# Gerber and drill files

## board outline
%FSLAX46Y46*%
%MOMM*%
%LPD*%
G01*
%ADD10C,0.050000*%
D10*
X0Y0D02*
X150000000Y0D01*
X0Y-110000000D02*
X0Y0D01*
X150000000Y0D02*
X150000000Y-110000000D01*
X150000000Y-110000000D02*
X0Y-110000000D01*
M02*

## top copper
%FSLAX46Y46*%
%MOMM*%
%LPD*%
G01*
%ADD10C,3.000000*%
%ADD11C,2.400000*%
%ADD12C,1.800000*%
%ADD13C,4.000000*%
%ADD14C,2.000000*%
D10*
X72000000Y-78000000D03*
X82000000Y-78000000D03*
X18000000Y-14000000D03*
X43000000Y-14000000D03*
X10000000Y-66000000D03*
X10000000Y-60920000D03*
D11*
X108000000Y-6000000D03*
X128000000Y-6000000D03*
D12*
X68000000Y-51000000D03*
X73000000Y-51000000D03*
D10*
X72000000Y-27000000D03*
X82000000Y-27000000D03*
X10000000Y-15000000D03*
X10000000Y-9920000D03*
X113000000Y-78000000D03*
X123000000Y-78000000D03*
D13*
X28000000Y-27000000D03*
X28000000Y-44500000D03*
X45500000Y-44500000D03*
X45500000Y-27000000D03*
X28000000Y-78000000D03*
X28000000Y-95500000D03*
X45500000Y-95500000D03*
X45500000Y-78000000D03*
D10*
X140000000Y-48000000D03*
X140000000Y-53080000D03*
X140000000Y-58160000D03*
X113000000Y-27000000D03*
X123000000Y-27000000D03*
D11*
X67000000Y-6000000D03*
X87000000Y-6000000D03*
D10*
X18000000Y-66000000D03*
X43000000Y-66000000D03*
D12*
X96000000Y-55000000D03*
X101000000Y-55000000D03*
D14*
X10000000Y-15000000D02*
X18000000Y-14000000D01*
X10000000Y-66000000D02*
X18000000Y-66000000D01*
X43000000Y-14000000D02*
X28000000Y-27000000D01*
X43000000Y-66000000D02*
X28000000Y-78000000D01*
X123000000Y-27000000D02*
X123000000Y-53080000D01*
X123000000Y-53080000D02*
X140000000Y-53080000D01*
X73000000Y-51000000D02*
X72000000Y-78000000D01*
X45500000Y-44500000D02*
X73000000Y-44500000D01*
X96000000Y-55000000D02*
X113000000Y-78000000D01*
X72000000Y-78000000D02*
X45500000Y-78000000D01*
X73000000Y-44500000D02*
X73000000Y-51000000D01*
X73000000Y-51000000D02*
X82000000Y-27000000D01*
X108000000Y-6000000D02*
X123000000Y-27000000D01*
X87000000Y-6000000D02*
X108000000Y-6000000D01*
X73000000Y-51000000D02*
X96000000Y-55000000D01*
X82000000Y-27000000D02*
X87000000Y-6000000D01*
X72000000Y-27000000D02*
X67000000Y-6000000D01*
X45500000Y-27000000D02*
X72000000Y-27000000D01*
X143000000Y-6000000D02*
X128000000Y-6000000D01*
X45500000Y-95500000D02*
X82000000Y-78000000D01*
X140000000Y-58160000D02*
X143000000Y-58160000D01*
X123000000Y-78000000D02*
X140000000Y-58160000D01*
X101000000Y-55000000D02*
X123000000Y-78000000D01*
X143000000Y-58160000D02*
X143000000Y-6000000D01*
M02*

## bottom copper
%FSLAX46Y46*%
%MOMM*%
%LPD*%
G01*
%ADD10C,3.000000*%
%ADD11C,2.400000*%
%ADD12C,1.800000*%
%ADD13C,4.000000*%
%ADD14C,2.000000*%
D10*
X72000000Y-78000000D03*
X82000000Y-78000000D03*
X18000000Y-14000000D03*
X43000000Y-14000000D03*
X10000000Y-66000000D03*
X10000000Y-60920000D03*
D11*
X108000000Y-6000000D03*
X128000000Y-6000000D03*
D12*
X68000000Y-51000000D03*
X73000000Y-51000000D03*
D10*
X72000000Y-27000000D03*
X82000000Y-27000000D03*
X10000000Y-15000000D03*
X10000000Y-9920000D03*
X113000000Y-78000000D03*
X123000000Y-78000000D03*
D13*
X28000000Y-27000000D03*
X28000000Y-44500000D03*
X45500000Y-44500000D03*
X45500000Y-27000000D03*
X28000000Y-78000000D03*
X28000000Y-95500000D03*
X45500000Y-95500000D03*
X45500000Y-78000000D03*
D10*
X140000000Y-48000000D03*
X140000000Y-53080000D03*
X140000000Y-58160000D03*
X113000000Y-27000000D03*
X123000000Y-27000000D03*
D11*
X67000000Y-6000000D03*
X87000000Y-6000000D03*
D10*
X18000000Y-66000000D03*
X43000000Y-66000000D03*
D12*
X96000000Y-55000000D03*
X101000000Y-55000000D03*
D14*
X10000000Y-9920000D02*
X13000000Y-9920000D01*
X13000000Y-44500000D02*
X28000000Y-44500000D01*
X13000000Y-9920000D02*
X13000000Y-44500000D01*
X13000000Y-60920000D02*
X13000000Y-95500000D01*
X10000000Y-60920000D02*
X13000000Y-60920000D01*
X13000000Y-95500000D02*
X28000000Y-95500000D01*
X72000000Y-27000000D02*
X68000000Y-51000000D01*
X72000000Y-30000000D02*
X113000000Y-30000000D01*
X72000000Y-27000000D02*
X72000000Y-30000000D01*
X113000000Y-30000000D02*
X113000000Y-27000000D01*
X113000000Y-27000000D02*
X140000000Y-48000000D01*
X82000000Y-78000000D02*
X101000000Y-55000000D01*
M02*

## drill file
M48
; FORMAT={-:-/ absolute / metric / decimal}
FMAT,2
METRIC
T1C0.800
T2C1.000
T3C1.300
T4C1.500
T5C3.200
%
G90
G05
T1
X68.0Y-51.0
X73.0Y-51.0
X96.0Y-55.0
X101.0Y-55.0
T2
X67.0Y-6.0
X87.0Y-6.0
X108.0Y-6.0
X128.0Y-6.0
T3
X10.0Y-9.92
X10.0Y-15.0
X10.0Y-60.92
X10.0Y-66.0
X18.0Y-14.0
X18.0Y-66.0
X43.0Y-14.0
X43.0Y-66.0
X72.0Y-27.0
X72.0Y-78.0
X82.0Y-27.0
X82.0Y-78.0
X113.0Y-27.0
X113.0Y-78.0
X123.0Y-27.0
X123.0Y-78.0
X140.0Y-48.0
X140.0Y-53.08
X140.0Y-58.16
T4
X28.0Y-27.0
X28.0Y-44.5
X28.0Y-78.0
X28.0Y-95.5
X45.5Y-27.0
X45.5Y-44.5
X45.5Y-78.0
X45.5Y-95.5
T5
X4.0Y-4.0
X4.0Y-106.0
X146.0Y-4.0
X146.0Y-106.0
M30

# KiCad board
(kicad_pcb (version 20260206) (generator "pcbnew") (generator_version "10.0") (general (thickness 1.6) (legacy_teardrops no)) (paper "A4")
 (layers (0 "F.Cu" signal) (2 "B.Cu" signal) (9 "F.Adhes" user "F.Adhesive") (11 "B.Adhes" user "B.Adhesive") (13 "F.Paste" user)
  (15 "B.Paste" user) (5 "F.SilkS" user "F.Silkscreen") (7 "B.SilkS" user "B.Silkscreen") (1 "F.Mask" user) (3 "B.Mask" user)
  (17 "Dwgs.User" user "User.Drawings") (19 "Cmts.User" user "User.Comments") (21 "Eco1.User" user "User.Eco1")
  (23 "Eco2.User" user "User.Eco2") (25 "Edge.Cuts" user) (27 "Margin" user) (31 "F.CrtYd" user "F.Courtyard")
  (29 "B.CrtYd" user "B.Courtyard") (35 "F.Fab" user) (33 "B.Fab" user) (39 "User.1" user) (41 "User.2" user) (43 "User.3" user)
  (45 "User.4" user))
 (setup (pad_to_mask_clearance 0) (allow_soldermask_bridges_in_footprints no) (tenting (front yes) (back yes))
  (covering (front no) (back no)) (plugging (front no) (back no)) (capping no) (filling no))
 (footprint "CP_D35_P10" (layer "F.Cu") (at 72 78)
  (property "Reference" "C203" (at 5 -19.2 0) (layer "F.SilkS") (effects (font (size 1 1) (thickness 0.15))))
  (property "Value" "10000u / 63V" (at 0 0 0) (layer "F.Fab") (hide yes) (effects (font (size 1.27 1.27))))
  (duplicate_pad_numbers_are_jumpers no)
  (pad "1" thru_hole circle (at 0 0) (size 3 3) (drill 1.3) (layers "*.Cu" "*.Mask") (remove_unused_layers no) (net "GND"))
  (pad "2" thru_hole circle (at 10 0) (size 3 3) (drill 1.3) (layers "*.Cu" "*.Mask") (remove_unused_layers no) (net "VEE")))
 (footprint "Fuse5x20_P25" (layer "F.Cu") (at 18 14)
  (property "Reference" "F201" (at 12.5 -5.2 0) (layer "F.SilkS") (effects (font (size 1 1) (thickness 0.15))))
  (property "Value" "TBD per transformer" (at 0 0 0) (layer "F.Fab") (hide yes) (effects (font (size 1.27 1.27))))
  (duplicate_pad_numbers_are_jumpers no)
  (pad "1" thru_hole circle (at 0 0) (size 3 3) (drill 1.3) (layers "*.Cu" "*.Mask") (remove_unused_layers no) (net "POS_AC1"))
  (pad "2" thru_hole circle (at 25 0) (size 3 3) (drill 1.3) (layers "*.Cu" "*.Mask") (remove_unused_layers no) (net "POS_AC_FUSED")))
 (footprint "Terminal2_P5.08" (layer "F.Cu") (at 10 66 90)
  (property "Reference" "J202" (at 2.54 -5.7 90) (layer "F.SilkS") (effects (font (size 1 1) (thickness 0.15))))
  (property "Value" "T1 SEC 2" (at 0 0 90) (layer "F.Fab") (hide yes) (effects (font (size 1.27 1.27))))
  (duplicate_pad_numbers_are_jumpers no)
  (pad "1" thru_hole circle (at 0 0 90) (size 3 3) (drill 1.3) (layers "*.Cu" "*.Mask") (remove_unused_layers no) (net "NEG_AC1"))
  (pad "2" thru_hole circle (at 5.08 0 90) (size 3 3) (drill 1.3) (layers "*.Cu" "*.Mask") (remove_unused_layers no) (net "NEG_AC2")))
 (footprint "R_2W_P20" (layer "F.Cu") (at 108 6)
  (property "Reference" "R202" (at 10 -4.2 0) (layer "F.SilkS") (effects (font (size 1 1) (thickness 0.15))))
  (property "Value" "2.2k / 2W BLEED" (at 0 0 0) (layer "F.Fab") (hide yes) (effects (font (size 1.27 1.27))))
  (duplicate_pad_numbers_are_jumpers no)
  (pad "1" thru_hole circle (at 0 0) (size 2.4 2.4) (drill 1) (layers "*.Cu" "*.Mask") (remove_unused_layers no) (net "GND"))
  (pad "2" thru_hole circle (at 20 0) (size 2.4 2.4) (drill 1) (layers "*.Cu" "*.Mask") (remove_unused_layers no) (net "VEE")))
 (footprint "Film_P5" (layer "F.Cu") (at 68 51)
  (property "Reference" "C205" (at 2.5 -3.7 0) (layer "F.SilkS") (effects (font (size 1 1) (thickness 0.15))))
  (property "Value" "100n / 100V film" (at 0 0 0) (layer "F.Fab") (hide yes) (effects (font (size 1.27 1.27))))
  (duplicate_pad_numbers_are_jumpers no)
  (pad "1" thru_hole circle (at 0 0) (size 1.8 1.8) (drill 0.8) (layers "*.Cu" "*.Mask") (remove_unused_layers no) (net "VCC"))
  (pad "2" thru_hole circle (at 5 0) (size 1.8 1.8) (drill 0.8) (layers "*.Cu" "*.Mask") (remove_unused_layers no) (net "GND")))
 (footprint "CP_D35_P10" (layer "F.Cu") (at 72 27)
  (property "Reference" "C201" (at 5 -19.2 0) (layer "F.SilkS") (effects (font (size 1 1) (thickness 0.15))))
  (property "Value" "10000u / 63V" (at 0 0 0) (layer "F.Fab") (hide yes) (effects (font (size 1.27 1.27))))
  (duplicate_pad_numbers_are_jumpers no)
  (pad "1" thru_hole circle (at 0 0) (size 3 3) (drill 1.3) (layers "*.Cu" "*.Mask") (remove_unused_layers no) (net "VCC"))
  (pad "2" thru_hole circle (at 10 0) (size 3 3) (drill 1.3) (layers "*.Cu" "*.Mask") (remove_unused_layers no) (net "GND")))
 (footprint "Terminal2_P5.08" (layer "F.Cu") (at 10 15 90)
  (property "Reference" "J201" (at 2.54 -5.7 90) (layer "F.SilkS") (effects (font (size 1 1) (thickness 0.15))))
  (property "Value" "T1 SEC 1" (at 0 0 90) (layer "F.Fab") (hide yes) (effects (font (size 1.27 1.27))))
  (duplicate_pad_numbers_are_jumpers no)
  (pad "1" thru_hole circle (at 0 0 90) (size 3 3) (drill 1.3) (layers "*.Cu" "*.Mask") (remove_unused_layers no) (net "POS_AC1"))
  (pad "2" thru_hole circle (at 5.08 0 90) (size 3 3) (drill 1.3) (layers "*.Cu" "*.Mask") (remove_unused_layers no) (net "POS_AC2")))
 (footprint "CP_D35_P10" (layer "F.Cu") (at 113 78)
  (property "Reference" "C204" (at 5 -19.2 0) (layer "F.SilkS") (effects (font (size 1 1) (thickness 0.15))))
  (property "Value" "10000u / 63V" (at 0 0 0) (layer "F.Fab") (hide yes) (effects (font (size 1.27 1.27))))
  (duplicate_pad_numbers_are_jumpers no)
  (pad "1" thru_hole circle (at 0 0) (size 3 3) (drill 1.3) (layers "*.Cu" "*.Mask") (remove_unused_layers no) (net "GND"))
  (pad "2" thru_hole circle (at 10 0) (size 3 3) (drill 1.3) (layers "*.Cu" "*.Mask") (remove_unused_layers no) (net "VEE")))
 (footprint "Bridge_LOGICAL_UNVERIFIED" (layer "F.Cu") (at 28 27)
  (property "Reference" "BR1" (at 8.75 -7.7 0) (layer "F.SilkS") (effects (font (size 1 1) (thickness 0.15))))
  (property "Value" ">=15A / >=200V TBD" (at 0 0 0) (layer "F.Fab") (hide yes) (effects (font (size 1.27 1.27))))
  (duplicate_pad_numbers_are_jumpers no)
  (pad "AC1" thru_hole circle (at 0 0) (size 4 4) (drill 1.5) (layers "*.Cu" "*.Mask") (remove_unused_layers no) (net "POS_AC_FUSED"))
  (pad "AC2" thru_hole circle (at 0 17.5) (size 4 4) (drill 1.5) (layers "*.Cu" "*.Mask") (remove_unused_layers no) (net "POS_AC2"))
  (pad "N" thru_hole circle (at 17.5 17.5) (size 4 4) (drill 1.5) (layers "*.Cu" "*.Mask") (remove_unused_layers no) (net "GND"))
  (pad "P" thru_hole circle (at 17.5 0) (size 4 4) (drill 1.5) (layers "*.Cu" "*.Mask") (remove_unused_layers no) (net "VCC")))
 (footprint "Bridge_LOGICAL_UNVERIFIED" (layer "F.Cu") (at 28 78)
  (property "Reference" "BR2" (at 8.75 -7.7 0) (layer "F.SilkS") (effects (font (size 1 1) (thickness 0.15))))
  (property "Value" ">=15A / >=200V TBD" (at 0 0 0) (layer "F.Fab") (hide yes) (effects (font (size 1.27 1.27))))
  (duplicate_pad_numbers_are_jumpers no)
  (pad "AC1" thru_hole circle (at 0 0) (size 4 4) (drill 1.5) (layers "*.Cu" "*.Mask") (remove_unused_layers no) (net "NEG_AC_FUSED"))
  (pad "AC2" thru_hole circle (at 0 17.5) (size 4 4) (drill 1.5) (layers "*.Cu" "*.Mask") (remove_unused_layers no) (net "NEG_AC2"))
  (pad "N" thru_hole circle (at 17.5 17.5) (size 4 4) (drill 1.5) (layers "*.Cu" "*.Mask") (remove_unused_layers no) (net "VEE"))
  (pad "P" thru_hole circle (at 17.5 0) (size 4 4) (drill 1.5) (layers "*.Cu" "*.Mask") (remove_unused_layers no) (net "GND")))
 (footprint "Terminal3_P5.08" (layer "F.Cu") (at 140 48 -90)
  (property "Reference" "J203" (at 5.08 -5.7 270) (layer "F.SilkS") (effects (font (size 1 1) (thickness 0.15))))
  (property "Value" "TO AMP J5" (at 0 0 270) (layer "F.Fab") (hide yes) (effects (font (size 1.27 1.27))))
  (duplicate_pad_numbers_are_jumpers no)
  (pad "1" thru_hole circle (at 0 0 270) (size 3 3) (drill 1.3) (layers "*.Cu" "*.Mask") (remove_unused_layers no) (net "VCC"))
  (pad "2" thru_hole circle (at 5.08 0 270) (size 3 3) (drill 1.3) (layers "*.Cu" "*.Mask") (remove_unused_layers no) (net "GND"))
  (pad "3" thru_hole circle (at 10.16 0 270) (size 3 3) (drill 1.3) (layers "*.Cu" "*.Mask") (remove_unused_layers no) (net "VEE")))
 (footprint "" (layer "F.Cu") (at 4 106)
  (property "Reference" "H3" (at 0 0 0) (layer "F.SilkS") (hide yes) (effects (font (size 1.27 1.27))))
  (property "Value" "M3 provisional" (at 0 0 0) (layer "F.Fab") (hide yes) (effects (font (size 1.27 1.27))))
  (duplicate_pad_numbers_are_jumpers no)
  (pad "" np_thru_hole circle (at 0 0) (size 3.2 3.2) (drill 3.2) (layers "*.Cu" "*.Mask")))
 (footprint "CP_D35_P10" (layer "F.Cu") (at 113 27)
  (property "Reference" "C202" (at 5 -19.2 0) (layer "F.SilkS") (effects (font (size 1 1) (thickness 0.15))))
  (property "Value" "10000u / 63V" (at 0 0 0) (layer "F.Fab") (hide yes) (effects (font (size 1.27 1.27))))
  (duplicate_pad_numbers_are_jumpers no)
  (pad "1" thru_hole circle (at 0 0) (size 3 3) (drill 1.3) (layers "*.Cu" "*.Mask") (remove_unused_layers no) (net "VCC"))
  (pad "2" thru_hole circle (at 10 0) (size 3 3) (drill 1.3) (layers "*.Cu" "*.Mask") (remove_unused_layers no) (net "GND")))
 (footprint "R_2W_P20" (layer "F.Cu") (at 67 6)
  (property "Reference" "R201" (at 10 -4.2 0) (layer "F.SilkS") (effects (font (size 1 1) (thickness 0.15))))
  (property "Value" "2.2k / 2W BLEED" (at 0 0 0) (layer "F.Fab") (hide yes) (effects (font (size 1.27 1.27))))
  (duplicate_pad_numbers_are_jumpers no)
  (pad "1" thru_hole circle (at 0 0) (size 2.4 2.4) (drill 1) (layers "*.Cu" "*.Mask") (remove_unused_layers no) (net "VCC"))
  (pad "2" thru_hole circle (at 20 0) (size 2.4 2.4) (drill 1) (layers "*.Cu" "*.Mask") (remove_unused_layers no) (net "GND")))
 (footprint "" (layer "F.Cu") (at 146 4)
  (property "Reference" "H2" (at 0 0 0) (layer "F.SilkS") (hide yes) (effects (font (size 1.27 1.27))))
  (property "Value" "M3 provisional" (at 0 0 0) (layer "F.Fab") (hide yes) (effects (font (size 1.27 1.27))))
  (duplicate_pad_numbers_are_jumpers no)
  (pad "" np_thru_hole circle (at 0 0) (size 3.2 3.2) (drill 3.2) (layers "*.Cu" "*.Mask")))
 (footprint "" (layer "F.Cu") (at 146 106)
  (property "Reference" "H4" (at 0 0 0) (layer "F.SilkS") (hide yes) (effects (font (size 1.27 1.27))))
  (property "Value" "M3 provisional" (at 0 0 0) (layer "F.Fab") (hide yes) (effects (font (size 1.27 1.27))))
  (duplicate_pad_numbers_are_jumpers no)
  (pad "" np_thru_hole circle (at 0 0) (size 3.2 3.2) (drill 3.2) (layers "*.Cu" "*.Mask")))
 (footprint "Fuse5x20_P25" (layer "F.Cu") (at 18 66)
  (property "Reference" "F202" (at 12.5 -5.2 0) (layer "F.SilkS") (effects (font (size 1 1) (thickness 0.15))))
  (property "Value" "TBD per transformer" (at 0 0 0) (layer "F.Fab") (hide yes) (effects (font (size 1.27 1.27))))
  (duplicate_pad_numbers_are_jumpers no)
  (pad "1" thru_hole circle (at 0 0) (size 3 3) (drill 1.3) (layers "*.Cu" "*.Mask") (remove_unused_layers no) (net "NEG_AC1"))
  (pad "2" thru_hole circle (at 25 0) (size 3 3) (drill 1.3) (layers "*.Cu" "*.Mask") (remove_unused_layers no) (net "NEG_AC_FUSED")))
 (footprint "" (layer "F.Cu") (at 4 4)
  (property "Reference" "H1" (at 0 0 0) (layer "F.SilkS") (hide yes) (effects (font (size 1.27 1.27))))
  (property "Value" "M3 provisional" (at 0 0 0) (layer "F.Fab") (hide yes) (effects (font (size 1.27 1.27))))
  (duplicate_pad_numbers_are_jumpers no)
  (pad "" np_thru_hole circle (at 0 0) (size 3.2 3.2) (drill 3.2) (layers "*.Cu" "*.Mask")))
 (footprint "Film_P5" (layer "F.Cu") (at 96 55)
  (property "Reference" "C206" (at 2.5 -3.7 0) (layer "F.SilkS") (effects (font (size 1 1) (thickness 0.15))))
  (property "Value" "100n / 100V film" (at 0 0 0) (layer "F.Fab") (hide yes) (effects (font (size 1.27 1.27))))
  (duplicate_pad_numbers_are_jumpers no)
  (pad "1" thru_hole circle (at 0 0) (size 1.8 1.8) (drill 0.8) (layers "*.Cu" "*.Mask") (remove_unused_layers no) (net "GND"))
  (pad "2" thru_hole circle (at 5 0) (size 1.8 1.8) (drill 0.8) (layers "*.Cu" "*.Mask") (remove_unused_layers no) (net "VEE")))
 (gr_line (start 0 0) (end 150 0) (stroke (width 0.05) (type default)) (layer "Edge.Cuts"))
 (gr_line (start 0 110) (end 0 0) (stroke (width 0.05) (type default)) (layer "Edge.Cuts"))
 (gr_line (start 150 0) (end 150 110) (stroke (width 0.05) (type default)) (layer "Edge.Cuts"))
 (gr_line (start 150 110) (end 0 110) (stroke (width 0.05) (type default)) (layer "Edge.Cuts"))
 (segment (start 10 15) (end 18 14) (width 2) (layer "F.Cu") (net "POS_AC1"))
 (segment (start 10 9.92) (end 13 9.92) (width 2) (layer "B.Cu") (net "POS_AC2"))
 (segment (start 13 44.5) (end 28 44.5) (width 2) (layer "B.Cu") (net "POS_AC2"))
 (segment (start 13 9.92) (end 13 44.5) (width 2) (layer "B.Cu") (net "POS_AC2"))
 (segment (start 10 66) (end 18 66) (width 2) (layer "F.Cu") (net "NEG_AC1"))
 (segment (start 13 60.92) (end 13 95.5) (width 2) (layer "B.Cu") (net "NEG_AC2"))
 (segment (start 10 60.92) (end 13 60.92) (width 2) (layer "B.Cu") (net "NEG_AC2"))
 (segment (start 13 95.5) (end 28 95.5) (width 2) (layer "B.Cu") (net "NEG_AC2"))
 (segment (start 43 14) (end 28 27) (width 2) (layer "F.Cu") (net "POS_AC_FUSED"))
 (segment (start 43 66) (end 28 78) (width 2) (layer "F.Cu") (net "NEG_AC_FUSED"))
 (segment (start 123 27) (end 123 53.08) (width 2) (layer "F.Cu") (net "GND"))
 (segment (start 123 53.08) (end 140 53.08) (width 2) (layer "F.Cu") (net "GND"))
 (segment (start 73 51) (end 72 78) (width 2) (layer "F.Cu") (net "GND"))
 (segment (start 45.5 44.5) (end 73 44.5) (width 2) (layer "F.Cu") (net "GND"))
 (segment (start 96 55) (end 113 78) (width 2) (layer "F.Cu") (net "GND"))
 (segment (start 72 78) (end 45.5 78) (width 2) (layer "F.Cu") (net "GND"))
 (segment (start 73 44.5) (end 73 51) (width 2) (layer "F.Cu") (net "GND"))
 (segment (start 73 51) (end 82 27) (width 2) (layer "F.Cu") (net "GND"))
 (segment (start 108 6) (end 123 27) (width 2) (layer "F.Cu") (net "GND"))
 (segment (start 87 6) (end 108 6) (width 2) (layer "F.Cu") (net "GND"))
 (segment (start 73 51) (end 96 55) (width 2) (layer "F.Cu") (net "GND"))
 (segment (start 82 27) (end 87 6) (width 2) (layer "F.Cu") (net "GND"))
 (segment (start 72 27) (end 67 6) (width 2) (layer "F.Cu") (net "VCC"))
 (segment (start 45.5 27) (end 72 27) (width 2) (layer "F.Cu") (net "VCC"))
 (segment (start 72 27) (end 68 51) (width 2) (layer "B.Cu") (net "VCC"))
 (segment (start 72 30) (end 113 30) (width 2) (layer "B.Cu") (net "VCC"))
 (segment (start 72 27) (end 72 30) (width 2) (layer "B.Cu") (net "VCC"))
 (segment (start 113 30) (end 113 27) (width 2) (layer "B.Cu") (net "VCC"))
 (segment (start 113 27) (end 140 48) (width 2) (layer "B.Cu") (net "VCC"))
 (segment (start 143 6) (end 128 6) (width 2) (layer "F.Cu") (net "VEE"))
 (segment (start 45.5 95.5) (end 82 78) (width 2) (layer "F.Cu") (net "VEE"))
 (segment (start 140 58.16) (end 143 58.16) (width 2) (layer "F.Cu") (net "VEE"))
 (segment (start 123 78) (end 140 58.16) (width 2) (layer "F.Cu") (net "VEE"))
 (segment (start 101 55) (end 123 78) (width 2) (layer "F.Cu") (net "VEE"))
 (segment (start 143 58.16) (end 143 6) (width 2) (layer "F.Cu") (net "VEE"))
 (segment (start 82 78) (end 101 55) (width 2) (layer "B.Cu") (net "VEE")))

